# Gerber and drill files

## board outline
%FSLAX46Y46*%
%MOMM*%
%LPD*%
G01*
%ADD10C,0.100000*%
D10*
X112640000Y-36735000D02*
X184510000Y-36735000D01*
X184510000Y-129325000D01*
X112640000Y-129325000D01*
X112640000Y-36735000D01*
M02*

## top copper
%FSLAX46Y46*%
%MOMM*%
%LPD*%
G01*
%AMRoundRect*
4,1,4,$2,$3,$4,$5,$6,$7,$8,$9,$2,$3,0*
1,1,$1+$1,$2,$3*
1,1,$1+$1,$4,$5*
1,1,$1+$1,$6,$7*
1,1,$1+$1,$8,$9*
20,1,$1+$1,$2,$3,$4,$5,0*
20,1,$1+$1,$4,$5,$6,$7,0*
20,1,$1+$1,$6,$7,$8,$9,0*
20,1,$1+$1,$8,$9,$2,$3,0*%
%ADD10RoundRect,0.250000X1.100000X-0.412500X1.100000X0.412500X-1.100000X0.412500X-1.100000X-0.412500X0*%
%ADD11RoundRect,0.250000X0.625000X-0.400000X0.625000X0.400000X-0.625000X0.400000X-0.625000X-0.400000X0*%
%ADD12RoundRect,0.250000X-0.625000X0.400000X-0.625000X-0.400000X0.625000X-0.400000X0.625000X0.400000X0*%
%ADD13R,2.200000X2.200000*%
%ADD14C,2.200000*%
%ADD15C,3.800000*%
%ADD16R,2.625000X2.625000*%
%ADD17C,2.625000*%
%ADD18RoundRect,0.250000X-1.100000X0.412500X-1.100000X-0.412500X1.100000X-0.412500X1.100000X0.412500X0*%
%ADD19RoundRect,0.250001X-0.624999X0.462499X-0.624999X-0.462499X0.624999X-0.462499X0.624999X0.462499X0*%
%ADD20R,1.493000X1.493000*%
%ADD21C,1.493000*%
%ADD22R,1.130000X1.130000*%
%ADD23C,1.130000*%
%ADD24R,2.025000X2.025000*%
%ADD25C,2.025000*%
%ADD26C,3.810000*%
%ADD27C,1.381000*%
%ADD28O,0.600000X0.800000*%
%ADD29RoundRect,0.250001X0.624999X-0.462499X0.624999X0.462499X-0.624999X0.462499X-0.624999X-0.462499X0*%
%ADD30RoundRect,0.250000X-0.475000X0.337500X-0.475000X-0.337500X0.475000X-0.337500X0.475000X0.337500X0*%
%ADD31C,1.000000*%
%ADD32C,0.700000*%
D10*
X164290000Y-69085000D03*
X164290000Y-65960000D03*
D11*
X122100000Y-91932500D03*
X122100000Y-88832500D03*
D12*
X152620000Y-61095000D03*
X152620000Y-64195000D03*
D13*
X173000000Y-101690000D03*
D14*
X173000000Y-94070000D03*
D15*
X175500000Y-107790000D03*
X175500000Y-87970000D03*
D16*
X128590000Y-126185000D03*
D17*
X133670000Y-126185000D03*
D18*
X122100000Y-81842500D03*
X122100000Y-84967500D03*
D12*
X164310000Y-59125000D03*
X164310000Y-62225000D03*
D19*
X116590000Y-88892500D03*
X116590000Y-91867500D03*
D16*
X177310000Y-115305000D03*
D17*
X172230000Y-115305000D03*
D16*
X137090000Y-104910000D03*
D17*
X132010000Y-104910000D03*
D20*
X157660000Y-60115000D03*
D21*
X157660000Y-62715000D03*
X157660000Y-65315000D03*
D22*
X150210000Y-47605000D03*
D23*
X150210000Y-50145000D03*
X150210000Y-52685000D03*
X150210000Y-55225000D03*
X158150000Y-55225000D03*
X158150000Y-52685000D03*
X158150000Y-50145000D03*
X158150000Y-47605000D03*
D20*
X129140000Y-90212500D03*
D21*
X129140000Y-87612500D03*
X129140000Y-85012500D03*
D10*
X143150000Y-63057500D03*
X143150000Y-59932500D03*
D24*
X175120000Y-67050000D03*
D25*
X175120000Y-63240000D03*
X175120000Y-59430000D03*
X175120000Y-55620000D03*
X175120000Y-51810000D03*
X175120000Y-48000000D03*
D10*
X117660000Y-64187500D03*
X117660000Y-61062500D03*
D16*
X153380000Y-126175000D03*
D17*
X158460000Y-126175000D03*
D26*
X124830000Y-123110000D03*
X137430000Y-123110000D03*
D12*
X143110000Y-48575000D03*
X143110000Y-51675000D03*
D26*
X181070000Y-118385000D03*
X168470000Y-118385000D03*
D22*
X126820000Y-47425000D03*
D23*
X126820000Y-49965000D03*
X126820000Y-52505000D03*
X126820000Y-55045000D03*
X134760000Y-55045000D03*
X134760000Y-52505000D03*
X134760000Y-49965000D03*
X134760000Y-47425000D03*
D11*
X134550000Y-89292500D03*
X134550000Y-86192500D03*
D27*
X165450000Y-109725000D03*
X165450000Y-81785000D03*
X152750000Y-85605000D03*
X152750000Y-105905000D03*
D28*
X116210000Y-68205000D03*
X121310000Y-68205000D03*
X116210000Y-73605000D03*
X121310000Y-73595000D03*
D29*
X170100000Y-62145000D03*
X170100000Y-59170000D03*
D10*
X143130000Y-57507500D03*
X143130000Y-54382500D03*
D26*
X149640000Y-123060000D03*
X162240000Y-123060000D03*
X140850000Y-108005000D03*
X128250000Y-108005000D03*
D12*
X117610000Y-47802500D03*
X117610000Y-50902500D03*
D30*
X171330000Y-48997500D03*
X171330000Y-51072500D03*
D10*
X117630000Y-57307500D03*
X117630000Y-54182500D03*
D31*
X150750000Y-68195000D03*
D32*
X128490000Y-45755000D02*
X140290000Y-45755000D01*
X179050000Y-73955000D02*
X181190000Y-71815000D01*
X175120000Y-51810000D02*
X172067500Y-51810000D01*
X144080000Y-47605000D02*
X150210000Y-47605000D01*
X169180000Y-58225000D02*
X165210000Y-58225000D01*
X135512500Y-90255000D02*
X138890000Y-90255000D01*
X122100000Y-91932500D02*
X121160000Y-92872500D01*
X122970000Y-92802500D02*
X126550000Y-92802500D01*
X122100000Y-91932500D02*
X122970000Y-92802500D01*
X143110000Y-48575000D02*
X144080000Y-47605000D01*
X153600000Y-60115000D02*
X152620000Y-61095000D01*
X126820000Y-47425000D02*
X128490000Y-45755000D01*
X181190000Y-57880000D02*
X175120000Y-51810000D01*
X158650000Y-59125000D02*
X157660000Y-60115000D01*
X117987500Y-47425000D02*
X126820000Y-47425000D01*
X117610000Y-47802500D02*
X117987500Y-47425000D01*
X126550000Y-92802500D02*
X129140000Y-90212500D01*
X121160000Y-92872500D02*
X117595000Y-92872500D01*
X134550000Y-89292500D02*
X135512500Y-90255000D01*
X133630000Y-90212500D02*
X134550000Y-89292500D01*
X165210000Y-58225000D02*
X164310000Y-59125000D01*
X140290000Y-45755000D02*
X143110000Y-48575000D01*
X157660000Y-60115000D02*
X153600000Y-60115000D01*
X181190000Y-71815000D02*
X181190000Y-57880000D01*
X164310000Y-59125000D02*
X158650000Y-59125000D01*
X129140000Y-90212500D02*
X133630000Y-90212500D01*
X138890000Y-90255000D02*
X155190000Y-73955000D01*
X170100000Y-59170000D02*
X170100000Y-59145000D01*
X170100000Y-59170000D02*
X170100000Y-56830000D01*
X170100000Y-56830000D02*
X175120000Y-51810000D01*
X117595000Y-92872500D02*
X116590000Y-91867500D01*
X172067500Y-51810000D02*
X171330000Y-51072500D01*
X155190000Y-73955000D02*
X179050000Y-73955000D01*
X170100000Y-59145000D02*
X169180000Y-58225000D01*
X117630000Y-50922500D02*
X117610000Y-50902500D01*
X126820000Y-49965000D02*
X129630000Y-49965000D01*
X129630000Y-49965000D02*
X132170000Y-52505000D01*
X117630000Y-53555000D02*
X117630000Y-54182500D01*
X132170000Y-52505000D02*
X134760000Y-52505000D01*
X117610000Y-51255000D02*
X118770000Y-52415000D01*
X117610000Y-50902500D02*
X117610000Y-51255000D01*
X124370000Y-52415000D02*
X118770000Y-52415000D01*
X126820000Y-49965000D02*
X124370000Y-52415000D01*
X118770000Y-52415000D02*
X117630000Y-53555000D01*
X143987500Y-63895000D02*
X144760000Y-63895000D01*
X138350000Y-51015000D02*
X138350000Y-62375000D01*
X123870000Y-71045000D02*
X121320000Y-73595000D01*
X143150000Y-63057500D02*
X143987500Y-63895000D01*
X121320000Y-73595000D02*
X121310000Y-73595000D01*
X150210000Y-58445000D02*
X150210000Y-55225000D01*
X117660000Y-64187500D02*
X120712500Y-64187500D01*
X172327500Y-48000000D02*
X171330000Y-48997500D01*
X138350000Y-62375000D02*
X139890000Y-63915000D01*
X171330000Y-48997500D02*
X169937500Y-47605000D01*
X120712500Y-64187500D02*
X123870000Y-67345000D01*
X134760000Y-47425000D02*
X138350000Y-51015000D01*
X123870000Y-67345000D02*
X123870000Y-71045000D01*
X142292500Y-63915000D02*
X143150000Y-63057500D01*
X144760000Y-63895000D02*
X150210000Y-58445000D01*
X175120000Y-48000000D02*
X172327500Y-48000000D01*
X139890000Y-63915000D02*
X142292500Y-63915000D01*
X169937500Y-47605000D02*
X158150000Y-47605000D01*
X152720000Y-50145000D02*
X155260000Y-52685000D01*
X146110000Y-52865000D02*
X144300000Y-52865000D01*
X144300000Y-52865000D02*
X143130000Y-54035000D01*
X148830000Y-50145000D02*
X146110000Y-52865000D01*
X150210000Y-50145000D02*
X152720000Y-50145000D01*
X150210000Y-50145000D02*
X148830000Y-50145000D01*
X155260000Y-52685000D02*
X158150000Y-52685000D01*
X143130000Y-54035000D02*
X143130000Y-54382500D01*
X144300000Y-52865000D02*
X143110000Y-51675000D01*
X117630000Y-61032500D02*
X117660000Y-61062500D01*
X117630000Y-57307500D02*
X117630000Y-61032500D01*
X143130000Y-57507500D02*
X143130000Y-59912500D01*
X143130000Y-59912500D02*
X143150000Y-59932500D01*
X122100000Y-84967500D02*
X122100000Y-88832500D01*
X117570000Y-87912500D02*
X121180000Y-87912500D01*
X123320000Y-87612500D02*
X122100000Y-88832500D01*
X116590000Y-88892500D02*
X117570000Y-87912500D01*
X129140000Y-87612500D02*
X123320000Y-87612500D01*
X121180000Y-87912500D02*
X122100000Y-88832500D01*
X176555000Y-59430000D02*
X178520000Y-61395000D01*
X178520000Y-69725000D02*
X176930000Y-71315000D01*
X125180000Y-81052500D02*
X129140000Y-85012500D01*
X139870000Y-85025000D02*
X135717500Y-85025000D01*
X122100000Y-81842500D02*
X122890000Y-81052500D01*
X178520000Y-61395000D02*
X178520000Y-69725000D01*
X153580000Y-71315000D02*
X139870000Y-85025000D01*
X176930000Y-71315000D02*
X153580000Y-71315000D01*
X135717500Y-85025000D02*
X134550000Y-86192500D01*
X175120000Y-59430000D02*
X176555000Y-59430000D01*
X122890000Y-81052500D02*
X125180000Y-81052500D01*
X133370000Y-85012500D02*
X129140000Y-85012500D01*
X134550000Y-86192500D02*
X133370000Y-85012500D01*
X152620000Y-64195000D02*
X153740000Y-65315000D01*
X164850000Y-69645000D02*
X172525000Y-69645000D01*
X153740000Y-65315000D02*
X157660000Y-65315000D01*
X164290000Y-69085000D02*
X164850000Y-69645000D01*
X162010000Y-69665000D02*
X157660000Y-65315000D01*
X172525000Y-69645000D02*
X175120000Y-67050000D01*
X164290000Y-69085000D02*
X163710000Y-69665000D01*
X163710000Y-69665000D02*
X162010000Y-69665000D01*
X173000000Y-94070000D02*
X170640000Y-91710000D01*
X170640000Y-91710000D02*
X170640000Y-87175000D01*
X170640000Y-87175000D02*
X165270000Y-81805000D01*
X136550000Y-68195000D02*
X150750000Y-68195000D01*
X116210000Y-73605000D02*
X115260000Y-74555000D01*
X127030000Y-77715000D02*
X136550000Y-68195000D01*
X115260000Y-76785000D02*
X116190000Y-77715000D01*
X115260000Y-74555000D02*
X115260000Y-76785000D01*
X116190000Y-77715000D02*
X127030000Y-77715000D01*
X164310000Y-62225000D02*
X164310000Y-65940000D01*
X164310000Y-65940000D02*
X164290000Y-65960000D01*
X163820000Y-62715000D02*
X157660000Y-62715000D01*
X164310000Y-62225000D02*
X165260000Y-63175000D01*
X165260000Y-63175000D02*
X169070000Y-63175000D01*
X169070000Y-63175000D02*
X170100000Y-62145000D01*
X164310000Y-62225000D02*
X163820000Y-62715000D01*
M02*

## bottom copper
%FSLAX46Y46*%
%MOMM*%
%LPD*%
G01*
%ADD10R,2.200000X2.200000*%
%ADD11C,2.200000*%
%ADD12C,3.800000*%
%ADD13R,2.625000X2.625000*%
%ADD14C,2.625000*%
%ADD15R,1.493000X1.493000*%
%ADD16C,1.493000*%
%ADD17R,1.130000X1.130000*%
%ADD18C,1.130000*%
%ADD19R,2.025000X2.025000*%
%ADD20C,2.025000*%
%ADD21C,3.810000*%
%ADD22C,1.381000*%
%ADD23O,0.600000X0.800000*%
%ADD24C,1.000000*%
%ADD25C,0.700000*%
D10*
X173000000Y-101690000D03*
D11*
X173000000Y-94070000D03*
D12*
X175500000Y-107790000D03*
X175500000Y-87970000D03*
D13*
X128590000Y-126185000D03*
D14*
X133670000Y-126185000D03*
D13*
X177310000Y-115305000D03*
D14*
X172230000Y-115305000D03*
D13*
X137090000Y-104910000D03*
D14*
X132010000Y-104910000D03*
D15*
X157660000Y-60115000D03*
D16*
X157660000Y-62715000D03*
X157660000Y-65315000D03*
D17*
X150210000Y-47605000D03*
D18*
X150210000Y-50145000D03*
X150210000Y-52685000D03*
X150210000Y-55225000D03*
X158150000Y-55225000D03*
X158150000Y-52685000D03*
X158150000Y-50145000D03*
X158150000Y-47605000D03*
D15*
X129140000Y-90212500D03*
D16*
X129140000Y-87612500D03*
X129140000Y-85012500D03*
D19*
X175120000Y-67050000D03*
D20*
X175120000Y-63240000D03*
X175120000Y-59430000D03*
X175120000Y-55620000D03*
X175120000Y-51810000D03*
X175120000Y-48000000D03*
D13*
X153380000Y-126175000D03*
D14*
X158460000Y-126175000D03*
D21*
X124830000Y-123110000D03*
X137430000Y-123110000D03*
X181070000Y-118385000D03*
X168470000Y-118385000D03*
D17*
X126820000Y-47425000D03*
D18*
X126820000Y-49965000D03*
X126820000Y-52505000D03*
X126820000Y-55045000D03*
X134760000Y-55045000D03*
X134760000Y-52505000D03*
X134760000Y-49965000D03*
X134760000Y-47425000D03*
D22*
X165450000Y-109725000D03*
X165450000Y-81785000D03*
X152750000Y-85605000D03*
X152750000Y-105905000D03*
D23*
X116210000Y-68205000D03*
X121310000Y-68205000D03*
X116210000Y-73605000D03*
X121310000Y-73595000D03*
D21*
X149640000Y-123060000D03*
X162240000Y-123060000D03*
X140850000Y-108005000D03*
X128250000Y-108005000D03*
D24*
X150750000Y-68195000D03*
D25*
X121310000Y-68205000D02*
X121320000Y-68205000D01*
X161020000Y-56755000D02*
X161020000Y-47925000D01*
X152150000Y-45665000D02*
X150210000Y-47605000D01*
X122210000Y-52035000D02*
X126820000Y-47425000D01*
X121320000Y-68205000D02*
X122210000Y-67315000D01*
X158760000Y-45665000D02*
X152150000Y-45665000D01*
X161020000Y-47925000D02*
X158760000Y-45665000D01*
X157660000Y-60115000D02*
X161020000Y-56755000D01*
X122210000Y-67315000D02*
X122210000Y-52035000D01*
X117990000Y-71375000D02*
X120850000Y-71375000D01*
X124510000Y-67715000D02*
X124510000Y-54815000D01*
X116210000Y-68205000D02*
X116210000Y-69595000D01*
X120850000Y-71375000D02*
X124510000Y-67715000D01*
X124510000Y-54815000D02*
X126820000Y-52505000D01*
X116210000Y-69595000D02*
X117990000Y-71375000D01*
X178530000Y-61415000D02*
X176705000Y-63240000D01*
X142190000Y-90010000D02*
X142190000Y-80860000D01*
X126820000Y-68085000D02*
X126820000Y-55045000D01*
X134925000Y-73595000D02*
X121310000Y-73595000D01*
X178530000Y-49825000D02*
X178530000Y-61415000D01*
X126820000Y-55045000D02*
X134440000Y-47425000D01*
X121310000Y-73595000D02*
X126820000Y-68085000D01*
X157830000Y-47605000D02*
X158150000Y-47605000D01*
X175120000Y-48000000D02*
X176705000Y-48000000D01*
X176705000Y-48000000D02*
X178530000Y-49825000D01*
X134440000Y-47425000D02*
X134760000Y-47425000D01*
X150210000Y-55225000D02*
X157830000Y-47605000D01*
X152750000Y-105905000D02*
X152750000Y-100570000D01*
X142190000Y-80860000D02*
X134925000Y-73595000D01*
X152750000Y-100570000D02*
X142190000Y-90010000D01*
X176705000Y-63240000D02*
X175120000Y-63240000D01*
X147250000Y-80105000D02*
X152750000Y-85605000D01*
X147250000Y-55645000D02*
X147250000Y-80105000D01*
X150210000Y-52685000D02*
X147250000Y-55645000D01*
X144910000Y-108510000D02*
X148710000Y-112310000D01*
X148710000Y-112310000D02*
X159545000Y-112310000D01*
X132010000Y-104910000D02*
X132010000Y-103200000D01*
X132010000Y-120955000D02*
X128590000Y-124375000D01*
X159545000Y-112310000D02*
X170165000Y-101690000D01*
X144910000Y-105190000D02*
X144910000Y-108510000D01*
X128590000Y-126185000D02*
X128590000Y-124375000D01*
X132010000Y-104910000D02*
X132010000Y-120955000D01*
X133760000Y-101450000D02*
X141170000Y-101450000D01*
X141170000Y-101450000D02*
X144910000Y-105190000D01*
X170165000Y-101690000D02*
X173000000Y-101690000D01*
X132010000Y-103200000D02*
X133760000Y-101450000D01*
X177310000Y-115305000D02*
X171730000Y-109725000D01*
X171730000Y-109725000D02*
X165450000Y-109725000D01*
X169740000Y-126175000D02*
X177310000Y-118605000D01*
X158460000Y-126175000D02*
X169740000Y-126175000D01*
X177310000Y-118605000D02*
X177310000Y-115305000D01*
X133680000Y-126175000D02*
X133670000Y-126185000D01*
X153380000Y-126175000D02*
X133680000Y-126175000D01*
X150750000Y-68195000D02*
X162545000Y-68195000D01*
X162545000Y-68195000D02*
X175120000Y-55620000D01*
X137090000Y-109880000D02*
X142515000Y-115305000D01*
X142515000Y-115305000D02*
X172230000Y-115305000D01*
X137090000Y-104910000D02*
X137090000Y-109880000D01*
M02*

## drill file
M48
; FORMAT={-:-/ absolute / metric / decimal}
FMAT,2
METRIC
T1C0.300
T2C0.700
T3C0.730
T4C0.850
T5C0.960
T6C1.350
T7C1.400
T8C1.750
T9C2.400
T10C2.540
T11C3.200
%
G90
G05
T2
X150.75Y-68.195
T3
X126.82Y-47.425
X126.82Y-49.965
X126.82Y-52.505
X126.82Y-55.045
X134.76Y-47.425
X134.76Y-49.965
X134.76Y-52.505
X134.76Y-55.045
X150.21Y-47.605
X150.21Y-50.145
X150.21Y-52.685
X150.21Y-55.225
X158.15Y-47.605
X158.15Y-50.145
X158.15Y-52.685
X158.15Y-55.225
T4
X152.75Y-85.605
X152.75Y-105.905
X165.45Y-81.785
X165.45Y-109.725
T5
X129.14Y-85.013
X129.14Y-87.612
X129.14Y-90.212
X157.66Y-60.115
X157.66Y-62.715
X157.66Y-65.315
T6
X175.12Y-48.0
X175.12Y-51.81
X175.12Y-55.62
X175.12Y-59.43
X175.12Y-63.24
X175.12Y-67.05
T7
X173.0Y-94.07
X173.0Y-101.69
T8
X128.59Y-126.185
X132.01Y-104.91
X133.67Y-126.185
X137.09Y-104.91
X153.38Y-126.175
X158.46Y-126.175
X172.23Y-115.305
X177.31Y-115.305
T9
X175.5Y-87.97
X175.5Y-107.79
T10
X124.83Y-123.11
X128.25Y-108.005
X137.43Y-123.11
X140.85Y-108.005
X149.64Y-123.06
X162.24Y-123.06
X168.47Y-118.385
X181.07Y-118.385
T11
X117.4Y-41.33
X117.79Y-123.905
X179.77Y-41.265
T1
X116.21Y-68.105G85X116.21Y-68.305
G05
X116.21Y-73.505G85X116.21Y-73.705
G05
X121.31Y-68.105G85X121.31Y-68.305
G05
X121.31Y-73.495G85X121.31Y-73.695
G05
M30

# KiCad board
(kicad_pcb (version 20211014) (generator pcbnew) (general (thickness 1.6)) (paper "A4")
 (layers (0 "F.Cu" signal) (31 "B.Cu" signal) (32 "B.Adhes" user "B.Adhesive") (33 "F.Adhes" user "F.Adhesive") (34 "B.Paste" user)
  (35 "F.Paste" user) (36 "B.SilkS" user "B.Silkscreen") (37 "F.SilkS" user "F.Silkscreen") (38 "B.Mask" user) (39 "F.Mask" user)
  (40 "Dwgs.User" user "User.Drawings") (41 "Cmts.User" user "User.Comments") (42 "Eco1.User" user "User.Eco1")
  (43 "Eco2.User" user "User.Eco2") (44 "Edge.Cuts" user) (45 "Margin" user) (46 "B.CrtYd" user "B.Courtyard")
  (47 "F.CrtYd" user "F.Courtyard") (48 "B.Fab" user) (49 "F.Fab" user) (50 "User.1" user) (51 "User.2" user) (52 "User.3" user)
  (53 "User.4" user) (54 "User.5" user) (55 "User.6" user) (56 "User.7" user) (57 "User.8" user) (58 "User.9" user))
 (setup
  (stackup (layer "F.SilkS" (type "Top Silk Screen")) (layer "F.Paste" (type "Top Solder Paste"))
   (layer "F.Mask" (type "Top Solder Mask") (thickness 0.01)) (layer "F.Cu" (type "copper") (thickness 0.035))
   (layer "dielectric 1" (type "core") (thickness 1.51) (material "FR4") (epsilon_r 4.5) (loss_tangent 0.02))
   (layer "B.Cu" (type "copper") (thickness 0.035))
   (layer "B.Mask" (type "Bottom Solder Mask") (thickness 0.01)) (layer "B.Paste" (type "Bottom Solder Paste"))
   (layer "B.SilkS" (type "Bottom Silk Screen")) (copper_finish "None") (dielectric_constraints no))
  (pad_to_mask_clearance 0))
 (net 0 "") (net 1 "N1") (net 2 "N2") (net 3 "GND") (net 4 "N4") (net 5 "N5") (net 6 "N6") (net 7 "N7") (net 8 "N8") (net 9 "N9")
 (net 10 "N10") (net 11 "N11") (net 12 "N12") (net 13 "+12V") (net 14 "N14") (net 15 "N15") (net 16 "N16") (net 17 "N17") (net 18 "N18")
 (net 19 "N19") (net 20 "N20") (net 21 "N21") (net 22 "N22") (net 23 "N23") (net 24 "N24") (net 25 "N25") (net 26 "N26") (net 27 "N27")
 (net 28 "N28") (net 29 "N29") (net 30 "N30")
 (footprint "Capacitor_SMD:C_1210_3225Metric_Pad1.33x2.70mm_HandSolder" (layer "F.Cu") (at 164.29 67.5225 90)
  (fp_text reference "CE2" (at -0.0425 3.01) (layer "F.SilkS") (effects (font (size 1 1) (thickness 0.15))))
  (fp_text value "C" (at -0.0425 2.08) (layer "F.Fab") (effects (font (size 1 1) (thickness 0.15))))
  (pad "1" smd roundrect (at -1.5625 0 90) (size 1.325 2.7) (layers "F.Cu" "F.Paste" "F.Mask") (roundrect_rratio 0.1886792453) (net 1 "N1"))
  (pad "2" smd roundrect (at 1.5625 0 90) (size 1.325 2.7) (layers "F.Cu" "F.Paste" "F.Mask") (roundrect_rratio 0.1886792453) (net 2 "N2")))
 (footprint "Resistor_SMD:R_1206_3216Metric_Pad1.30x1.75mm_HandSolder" (layer "F.Cu") (at 122.1 90.3825 90)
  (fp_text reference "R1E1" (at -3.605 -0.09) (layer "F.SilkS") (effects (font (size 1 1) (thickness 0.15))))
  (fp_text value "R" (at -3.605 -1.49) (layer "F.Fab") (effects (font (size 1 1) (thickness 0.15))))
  (pad "1" smd roundrect (at -1.55 0 90) (size 1.3 1.75) (layers "F.Cu" "F.Paste" "F.Mask") (roundrect_rratio 0.1923076923) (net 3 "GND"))
  (pad "2" smd roundrect (at 1.55 0 90) (size 1.3 1.75) (layers "F.Cu" "F.Paste" "F.Mask") (roundrect_rratio 0.1923076923) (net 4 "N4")))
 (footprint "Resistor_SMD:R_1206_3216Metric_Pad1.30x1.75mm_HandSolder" (layer "F.Cu") (at 152.62 62.645 -90)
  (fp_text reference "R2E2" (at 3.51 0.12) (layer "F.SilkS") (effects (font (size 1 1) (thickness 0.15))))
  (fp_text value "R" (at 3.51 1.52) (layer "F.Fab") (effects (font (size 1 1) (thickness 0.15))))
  (pad "1" smd roundrect (at -1.55 0 270) (size 1.3 1.75) (layers "F.Cu" "F.Paste" "F.Mask") (roundrect_rratio 0.1923076923) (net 3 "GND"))
  (pad "2" smd roundrect (at 1.55 0 270) (size 1.3 1.75) (layers "F.Cu" "F.Paste" "F.Mask") (roundrect_rratio 0.1923076923) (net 1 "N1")))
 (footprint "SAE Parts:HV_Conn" (layer "F.Cu") (at 173 101.69 90)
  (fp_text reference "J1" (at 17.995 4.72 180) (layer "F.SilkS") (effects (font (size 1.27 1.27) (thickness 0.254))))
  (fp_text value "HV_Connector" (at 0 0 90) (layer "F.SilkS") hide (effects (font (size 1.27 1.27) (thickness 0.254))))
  (pad "1" thru_hole rect (at 0 0 90) (size 2.2 2.2) (drill 1.4) (layers *.Cu *.Mask) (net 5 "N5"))
  (pad "2" thru_hole circle (at 7.62 0 90) (size 2.2 2.2) (drill 1.4) (layers *.Cu *.Mask) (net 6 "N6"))
  (pad "3" thru_hole circle (at -6.1 2.5 90) (size 3.8 3.8) (drill 2.4) (layers *.Cu *.Mask))
  (pad "4" thru_hole circle (at 13.72 2.5 90) (size 3.8 3.8) (drill 2.4) (layers *.Cu *.Mask)))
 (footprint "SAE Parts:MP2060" (layer "F.Cu") (at 128.59 126.185)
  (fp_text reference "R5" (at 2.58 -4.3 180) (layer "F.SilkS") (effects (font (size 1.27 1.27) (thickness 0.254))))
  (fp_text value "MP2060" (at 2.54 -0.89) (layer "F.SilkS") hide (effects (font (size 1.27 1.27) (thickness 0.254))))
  (pad "1" thru_hole rect (at 0 0) (size 2.625 2.625) (drill 1.75) (layers *.Cu *.Mask) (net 5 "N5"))
  (pad "2" thru_hole circle (at 5.08 0) (size 2.625 2.625) (drill 1.75) (layers *.Cu *.Mask) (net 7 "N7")))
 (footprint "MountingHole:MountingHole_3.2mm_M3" (layer "F.Cu") (at 117.4 41.33)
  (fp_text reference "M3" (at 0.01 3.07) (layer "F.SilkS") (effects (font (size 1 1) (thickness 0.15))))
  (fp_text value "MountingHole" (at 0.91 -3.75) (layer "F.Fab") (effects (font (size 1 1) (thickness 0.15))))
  (pad "" np_thru_hole circle (at 0 0) (size 3.2 3.2) (drill 3.2) (layers *.Cu *.Mask)))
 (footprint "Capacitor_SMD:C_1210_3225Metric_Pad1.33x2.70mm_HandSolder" (layer "F.Cu") (at 122.1 83.405 -90)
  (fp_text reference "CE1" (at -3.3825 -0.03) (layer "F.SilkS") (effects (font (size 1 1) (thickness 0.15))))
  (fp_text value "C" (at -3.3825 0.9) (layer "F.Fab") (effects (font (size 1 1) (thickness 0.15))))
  (pad "1" smd roundrect (at -1.5625 0 270) (size 1.325 2.7) (layers "F.Cu" "F.Paste" "F.Mask") (roundrect_rratio 0.1886792453) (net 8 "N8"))
  (pad "2" smd roundrect (at 1.5625 0 270) (size 1.325 2.7) (layers "F.Cu" "F.Paste" "F.Mask") (roundrect_rratio 0.1886792453) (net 4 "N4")))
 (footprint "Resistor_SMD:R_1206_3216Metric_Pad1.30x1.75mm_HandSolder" (layer "F.Cu") (at 164.31 60.675 -90)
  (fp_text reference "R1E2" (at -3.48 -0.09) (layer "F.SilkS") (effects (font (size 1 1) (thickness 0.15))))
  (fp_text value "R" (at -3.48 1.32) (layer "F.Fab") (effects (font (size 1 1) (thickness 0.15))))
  (pad "1" smd roundrect (at -1.55 0 270) (size 1.3 1.75) (layers "F.Cu" "F.Paste" "F.Mask") (roundrect_rratio 0.1923076923) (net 3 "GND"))
  (pad "2" smd roundrect (at 1.55 0 270) (size 1.3 1.75) (layers "F.Cu" "F.Paste" "F.Mask") (roundrect_rratio 0.1923076923) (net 2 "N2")))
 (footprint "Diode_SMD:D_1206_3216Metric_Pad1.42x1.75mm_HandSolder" (layer "F.Cu") (at 116.59 90.38 -90)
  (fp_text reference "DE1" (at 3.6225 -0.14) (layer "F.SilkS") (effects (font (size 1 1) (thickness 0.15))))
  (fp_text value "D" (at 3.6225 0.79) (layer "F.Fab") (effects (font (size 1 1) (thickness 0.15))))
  (pad "1" smd roundrect (at -1.4875 0 270) (size 1.425 1.75) (layers "F.Cu" "F.Paste" "F.Mask") (roundrect_rratio 0.1754392982)
   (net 4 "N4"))
  (pad "2" smd roundrect (at 1.4875 0 270) (size 1.425 1.75) (layers "F.Cu" "F.Paste" "F.Mask") (roundrect_rratio 0.1754392982)
   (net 3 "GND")))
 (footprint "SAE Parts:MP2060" (layer "F.Cu") (at 177.31 115.305 180)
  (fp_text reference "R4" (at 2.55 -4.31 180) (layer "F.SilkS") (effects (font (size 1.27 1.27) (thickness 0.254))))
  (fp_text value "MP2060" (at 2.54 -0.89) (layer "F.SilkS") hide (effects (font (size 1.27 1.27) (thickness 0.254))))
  (pad "1" thru_hole rect (at 0 0 180) (size 2.625 2.625) (drill 1.75) (layers *.Cu *.Mask) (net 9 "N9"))
  (pad "2" thru_hole circle (at 5.08 0 180) (size 2.625 2.625) (drill 1.75) (layers *.Cu *.Mask) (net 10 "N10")))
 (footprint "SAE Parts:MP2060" (layer "F.Cu") (at 137.09 104.91 180)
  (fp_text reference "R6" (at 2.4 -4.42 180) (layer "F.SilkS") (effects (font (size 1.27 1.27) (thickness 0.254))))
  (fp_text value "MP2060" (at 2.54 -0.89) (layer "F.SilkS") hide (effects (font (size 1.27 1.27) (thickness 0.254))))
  (pad "1" thru_hole rect (at 0 0 180) (size 2.625 2.625) (drill 1.75) (layers *.Cu *.Mask) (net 10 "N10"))
  (pad "2" thru_hole circle (at 5.08 0 180) (size 2.625 2.625) (drill 1.75) (layers *.Cu *.Mask) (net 5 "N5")))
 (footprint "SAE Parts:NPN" (layer "F.Cu") (at 157.66 60.115 -90)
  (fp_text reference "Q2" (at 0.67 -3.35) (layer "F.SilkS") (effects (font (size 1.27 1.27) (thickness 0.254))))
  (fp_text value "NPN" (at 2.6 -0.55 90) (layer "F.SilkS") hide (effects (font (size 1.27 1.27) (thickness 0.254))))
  (pad "1" thru_hole rect (at 0 0 270) (size 1.493 1.493) (drill 0.96) (layers *.Cu *.Mask) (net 3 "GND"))
  (pad "2" thru_hole circle (at 2.6 0 270) (size 1.493 1.493) (drill 0.96) (layers *.Cu *.Mask) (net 2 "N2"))
  (pad "3" thru_hole circle (at 5.2 0 270) (size 1.493 1.493) (drill 0.96) (layers *.Cu *.Mask) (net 1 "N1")))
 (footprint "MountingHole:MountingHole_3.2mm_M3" (layer "F.Cu") (at 117.79 123.905)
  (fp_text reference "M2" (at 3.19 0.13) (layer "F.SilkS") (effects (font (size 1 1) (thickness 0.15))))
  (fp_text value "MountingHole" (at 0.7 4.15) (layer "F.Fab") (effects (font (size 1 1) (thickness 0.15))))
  (pad "" np_thru_hole circle (at 0 0) (size 3.2 3.2) (drill 3.2) (layers *.Cu *.Mask)))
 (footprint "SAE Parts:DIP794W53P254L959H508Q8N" (layer "F.Cu") (at 154.18 51.415)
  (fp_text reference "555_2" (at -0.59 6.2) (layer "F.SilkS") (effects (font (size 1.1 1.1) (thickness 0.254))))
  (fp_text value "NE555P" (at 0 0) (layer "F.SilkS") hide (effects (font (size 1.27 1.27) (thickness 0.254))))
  (pad "1" thru_hole rect (at -3.97 -3.81) (size 1.13 1.13) (drill 0.73) (layers *.Cu *.Mask) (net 3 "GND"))
  (pad "2" thru_hole circle (at -3.97 -1.27) (size 1.13 1.13) (drill 0.73) (layers *.Cu *.Mask) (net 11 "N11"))
  (pad "3" thru_hole circle (at -3.97 1.27) (size 1.13 1.13) (drill 0.73) (layers *.Cu *.Mask) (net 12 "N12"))
  (pad "4" thru_hole circle (at -3.97 3.81) (size 1.13 1.13) (drill 0.73) (layers *.Cu *.Mask) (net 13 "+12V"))
  (pad "5" thru_hole circle (at 3.97 3.81) (size 1.13 1.13) (drill 0.73) (layers *.Cu *.Mask) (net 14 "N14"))
  (pad "6" thru_hole circle (at 3.97 1.27) (size 1.13 1.13) (drill 0.73) (layers *.Cu *.Mask) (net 11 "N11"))
  (pad "7" thru_hole circle (at 3.97 -1.27) (size 1.13 1.13) (drill 0.73) (layers *.Cu *.Mask) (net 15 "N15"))
  (pad "8" thru_hole circle (at 3.97 -3.81) (size 1.13 1.13) (drill 0.73) (layers *.Cu *.Mask) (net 13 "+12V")))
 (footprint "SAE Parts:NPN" (layer "F.Cu") (at 129.14 90.2125 90)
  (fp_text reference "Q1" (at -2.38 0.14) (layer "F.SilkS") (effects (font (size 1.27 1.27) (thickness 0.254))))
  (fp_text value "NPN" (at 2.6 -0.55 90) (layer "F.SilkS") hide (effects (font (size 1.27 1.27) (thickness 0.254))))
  (pad "1" thru_hole rect (at 0 0 90) (size 1.493 1.493) (drill 0.96) (layers *.Cu *.Mask) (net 3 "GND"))
  (pad "2" thru_hole circle (at 2.6 0 90) (size 1.493 1.493) (drill 0.96) (layers *.Cu *.Mask) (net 4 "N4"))
  (pad "3" thru_hole circle (at 5.2 0 90) (size 1.493 1.493) (drill 0.96) (layers *.Cu *.Mask) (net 8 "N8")))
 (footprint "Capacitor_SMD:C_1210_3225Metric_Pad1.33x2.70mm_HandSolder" (layer "F.Cu") (at 143.15 61.495 90)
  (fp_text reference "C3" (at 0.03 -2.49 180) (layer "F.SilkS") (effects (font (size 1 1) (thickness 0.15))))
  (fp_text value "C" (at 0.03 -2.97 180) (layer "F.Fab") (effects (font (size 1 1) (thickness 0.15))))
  (pad "1" smd roundrect (at -1.5625 0 90) (size 1.325 2.7) (layers "F.Cu" "F.Paste" "F.Mask") (roundrect_rratio 0.1886792453)
   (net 13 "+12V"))
  (pad "2" smd roundrect (at 1.5625 0 90) (size 1.325 2.7) (layers "F.Cu" "F.Paste" "F.Mask") (roundrect_rratio 0.1886792453) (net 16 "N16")))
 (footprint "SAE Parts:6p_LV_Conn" (layer "F.Cu") (at 175.12 67.05 -90)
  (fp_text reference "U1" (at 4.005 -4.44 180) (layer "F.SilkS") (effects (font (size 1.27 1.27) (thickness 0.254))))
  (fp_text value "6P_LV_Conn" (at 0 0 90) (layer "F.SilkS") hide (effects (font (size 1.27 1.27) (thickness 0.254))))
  (pad "1" thru_hole rect (at 0 0 270) (size 2.025 2.025) (drill 1.35) (layers *.Cu *.Mask) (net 1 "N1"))
  (pad "2" thru_hole circle (at -3.81 0 270) (size 2.025 2.025) (drill 1.35) (layers *.Cu *.Mask) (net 13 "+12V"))
  (pad "3" thru_hole circle (at -7.62 0 270) (size 2.025 2.025) (drill 1.35) (layers *.Cu *.Mask) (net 8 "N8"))
  (pad "4" thru_hole circle (at -11.43 0 270) (size 2.025 2.025) (drill 1.35) (layers *.Cu *.Mask) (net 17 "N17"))
  (pad "5" thru_hole circle (at -15.24 0 270) (size 2.025 2.025) (drill 1.35) (layers *.Cu *.Mask) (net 3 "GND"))
  (pad "6" thru_hole circle (at -19.05 0 270) (size 2.025 2.025) (drill 1.35) (layers *.Cu *.Mask) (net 13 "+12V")))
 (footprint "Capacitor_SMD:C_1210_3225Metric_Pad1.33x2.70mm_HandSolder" (layer "F.Cu") (at 117.66 62.625 90)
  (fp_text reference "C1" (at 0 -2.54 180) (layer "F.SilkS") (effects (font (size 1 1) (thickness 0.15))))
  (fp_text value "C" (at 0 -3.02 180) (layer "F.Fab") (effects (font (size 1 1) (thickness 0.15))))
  (pad "1" smd roundrect (at -1.5625 0 90) (size 1.325 2.7) (layers "F.Cu" "F.Paste" "F.Mask") (roundrect_rratio 0.1886792453)
   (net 13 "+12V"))
  (pad "2" smd roundrect (at 1.5625 0 90) (size 1.325 2.7) (layers "F.Cu" "F.Paste" "F.Mask") (roundrect_rratio 0.1886792453) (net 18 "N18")))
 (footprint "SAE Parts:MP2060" (layer "F.Cu") (at 153.38 126.175)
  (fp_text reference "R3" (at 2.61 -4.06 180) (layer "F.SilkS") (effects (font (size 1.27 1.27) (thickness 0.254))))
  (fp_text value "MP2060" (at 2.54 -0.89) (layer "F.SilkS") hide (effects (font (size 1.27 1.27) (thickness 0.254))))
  (pad "1" thru_hole rect (at 0 0) (size 2.625 2.625) (drill 1.75) (layers *.Cu *.Mask) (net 7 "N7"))
  (pad "2" thru_hole circle (at 5.08 0) (size 2.625 2.625) (drill 1.75) (layers *.Cu *.Mask) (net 9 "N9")))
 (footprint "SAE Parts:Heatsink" (layer "F.Cu") (at 124.83 123.11)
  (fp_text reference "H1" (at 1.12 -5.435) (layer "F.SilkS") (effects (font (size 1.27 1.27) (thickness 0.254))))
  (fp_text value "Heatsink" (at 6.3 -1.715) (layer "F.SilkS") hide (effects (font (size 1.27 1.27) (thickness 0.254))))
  (pad "1" thru_hole circle (at 0 0) (size 3.81 3.81) (drill 2.54) (layers *.Cu *.Mask) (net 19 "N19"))
  (pad "2" thru_hole circle (at 12.6 0) (size 3.81 3.81) (drill 2.54) (layers *.Cu *.Mask) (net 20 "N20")))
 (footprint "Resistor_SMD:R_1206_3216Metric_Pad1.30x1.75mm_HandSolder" (layer "F.Cu") (at 143.11 50.125 -90)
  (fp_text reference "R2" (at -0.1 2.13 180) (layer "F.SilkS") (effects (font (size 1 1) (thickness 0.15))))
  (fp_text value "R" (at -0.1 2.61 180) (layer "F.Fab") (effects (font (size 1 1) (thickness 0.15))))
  (pad "1" smd roundrect (at -1.55 0 270) (size 1.3 1.75) (layers "F.Cu" "F.Paste" "F.Mask") (roundrect_rratio 0.1923076923) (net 3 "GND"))
  (pad "2" smd roundrect (at 1.55 0 270) (size 1.3 1.75) (layers "F.Cu" "F.Paste" "F.Mask") (roundrect_rratio 0.1923076923) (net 11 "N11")))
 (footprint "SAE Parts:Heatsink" (layer "F.Cu") (at 181.07 118.385 180)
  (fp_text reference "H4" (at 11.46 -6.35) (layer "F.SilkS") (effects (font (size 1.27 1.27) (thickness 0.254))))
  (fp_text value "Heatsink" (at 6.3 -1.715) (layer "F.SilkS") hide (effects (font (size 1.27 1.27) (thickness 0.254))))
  (pad "1" thru_hole circle (at 0 0 180) (size 3.81 3.81) (drill 2.54) (layers *.Cu *.Mask) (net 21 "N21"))
  (pad "2" thru_hole circle (at 12.6 0 180) (size 3.81 3.81) (drill 2.54) (layers *.Cu *.Mask) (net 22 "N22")))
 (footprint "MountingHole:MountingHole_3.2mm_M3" (layer "F.Cu") (at 179.77 41.265)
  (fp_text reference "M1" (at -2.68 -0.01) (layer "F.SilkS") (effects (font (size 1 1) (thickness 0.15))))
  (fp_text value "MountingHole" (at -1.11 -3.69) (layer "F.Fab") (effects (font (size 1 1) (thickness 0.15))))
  (pad "" np_thru_hole circle (at 0 0) (size 3.2 3.2) (drill 3.2) (layers *.Cu *.Mask)))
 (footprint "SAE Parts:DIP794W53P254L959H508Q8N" (layer "F.Cu") (at 130.79 51.235)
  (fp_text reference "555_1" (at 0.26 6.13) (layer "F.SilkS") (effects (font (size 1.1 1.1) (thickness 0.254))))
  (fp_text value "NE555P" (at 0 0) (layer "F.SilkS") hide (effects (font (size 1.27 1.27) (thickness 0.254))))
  (pad "1" thru_hole rect (at -3.97 -3.81) (size 1.13 1.13) (drill 0.73) (layers *.Cu *.Mask) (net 3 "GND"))
  (pad "2" thru_hole circle (at -3.97 -1.27) (size 1.13 1.13) (drill 0.73) (layers *.Cu *.Mask) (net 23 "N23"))
  (pad "3" thru_hole circle (at -3.97 1.27) (size 1.13 1.13) (drill 0.73) (layers *.Cu *.Mask) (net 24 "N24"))
  (pad "4" thru_hole circle (at -3.97 3.81) (size 1.13 1.13) (drill 0.73) (layers *.Cu *.Mask) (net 13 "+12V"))
  (pad "5" thru_hole circle (at 3.97 3.81) (size 1.13 1.13) (drill 0.73) (layers *.Cu *.Mask) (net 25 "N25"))
  (pad "6" thru_hole circle (at 3.97 1.27) (size 1.13 1.13) (drill 0.73) (layers *.Cu *.Mask) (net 23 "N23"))
  (pad "7" thru_hole circle (at 3.97 -1.27) (size 1.13 1.13) (drill 0.73) (layers *.Cu *.Mask) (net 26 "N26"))
  (pad "8" thru_hole circle (at 3.97 -3.81) (size 1.13 1.13) (drill 0.73) (layers *.Cu *.Mask) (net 13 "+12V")))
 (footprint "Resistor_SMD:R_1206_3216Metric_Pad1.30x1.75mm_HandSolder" (layer "F.Cu") (at 134.55 87.7425 90)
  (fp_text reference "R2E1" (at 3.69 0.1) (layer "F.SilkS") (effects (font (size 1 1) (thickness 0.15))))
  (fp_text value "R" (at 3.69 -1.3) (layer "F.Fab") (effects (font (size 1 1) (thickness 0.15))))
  (pad "1" smd roundrect (at -1.55 0 90) (size 1.3 1.75) (layers "F.Cu" "F.Paste" "F.Mask") (roundrect_rratio 0.1923076923) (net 3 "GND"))
  (pad "2" smd roundrect (at 1.55 0 90) (size 1.3 1.75) (layers "F.Cu" "F.Paste" "F.Mask") (roundrect_rratio 0.1923076923) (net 8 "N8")))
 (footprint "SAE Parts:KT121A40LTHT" (layer "F.Cu") (at 165.45 109.725 90)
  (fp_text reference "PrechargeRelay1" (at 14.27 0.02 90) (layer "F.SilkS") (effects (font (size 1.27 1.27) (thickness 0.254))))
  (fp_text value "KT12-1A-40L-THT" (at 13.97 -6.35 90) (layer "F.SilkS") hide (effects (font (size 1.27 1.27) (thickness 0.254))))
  (pad "1" thru_hole circle (at 0 0 90) (size 1.381 1.381) (drill 0.85) (layers *.Cu *.Mask) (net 9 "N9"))
  (pad "2" thru_hole circle (at 27.94 0 90) (size 1.381 1.381) (drill 0.85) (layers *.Cu *.Mask) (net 6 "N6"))
  (pad "3" thru_hole circle (at 24.12 -12.7 90) (size 1.381 1.381) (drill 0.85) (layers *.Cu *.Mask) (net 12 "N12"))
  (pad "4" thru_hole circle (at 3.82 -12.7 90) (size 1.381 1.381) (drill 0.85) (layers *.Cu *.Mask) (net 13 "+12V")))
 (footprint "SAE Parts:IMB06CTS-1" (layer "F.Cu") (at 118.91 72.105)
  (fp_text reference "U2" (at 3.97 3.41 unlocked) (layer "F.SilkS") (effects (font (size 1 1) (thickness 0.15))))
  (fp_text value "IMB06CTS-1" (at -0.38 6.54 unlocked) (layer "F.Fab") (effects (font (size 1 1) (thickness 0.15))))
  (pad "1" thru_hole oval (at -2.7 -3.9) (size 0.6 0.8) (drill oval 0.3 0.5) (layers *.Cu *.Mask) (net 24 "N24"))
  (pad "2" thru_hole oval (at 2.4 -3.9) (size 0.6 0.8) (drill oval 0.3 0.5) (layers *.Cu *.Mask) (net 3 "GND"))
  (pad "3" thru_hole oval (at -2.7 1.5) (size 0.6 0.8) (drill oval 0.3 0.5) (layers *.Cu *.Mask) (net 17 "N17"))
  (pad "4" thru_hole oval (at 2.4 1.49) (size 0.6 0.8) (drill oval 0.3 0.5) (layers *.Cu *.Mask) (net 13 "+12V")))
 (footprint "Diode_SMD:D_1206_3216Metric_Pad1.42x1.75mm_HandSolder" (layer "F.Cu") (at 170.1 60.6575 90)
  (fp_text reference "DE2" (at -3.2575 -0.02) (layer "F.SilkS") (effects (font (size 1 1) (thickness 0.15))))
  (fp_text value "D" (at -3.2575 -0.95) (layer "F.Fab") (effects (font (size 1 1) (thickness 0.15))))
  (pad "1" smd roundrect (at -1.4875 0 90) (size 1.425 1.75) (layers "F.Cu" "F.Paste" "F.Mask") (roundrect_rratio 0.1754392982) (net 2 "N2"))
  (pad "2" smd roundrect (at 1.4875 0 90) (size 1.425 1.75) (layers "F.Cu" "F.Paste" "F.Mask") (roundrect_rratio 0.1754392982) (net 3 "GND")))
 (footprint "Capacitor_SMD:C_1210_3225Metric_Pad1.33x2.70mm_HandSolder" (layer "F.Cu") (at 143.13 55.945 90)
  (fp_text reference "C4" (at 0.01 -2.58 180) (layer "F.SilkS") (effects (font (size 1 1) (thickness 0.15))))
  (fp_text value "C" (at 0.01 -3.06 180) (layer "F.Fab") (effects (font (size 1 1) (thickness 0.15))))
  (pad "1" smd roundrect (at -1.5625 0 90) (size 1.325 2.7) (layers "F.Cu" "F.Paste" "F.Mask") (roundrect_rratio 0.1886792453)
   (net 16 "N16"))
  (pad "2" smd roundrect (at 1.5625 0 90) (size 1.325 2.7) (layers "F.Cu" "F.Paste" "F.Mask") (roundrect_rratio 0.1886792453) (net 11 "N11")))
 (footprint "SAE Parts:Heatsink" (layer "F.Cu") (at 149.64 123.06)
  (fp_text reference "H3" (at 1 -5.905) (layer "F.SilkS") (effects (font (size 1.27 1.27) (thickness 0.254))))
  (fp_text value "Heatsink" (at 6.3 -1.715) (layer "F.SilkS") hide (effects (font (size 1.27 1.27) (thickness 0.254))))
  (pad "1" thru_hole circle (at 0 0) (size 3.81 3.81) (drill 2.54) (layers *.Cu *.Mask) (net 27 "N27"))
  (pad "2" thru_hole circle (at 12.6 0) (size 3.81 3.81) (drill 2.54) (layers *.Cu *.Mask) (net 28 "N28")))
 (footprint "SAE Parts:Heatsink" (layer "F.Cu") (at 140.85 108.005 180)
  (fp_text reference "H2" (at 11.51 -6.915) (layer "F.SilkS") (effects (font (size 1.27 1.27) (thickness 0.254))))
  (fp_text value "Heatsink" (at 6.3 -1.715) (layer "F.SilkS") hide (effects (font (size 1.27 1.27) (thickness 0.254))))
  (pad "1" thru_hole circle (at 0 0 180) (size 3.81 3.81) (drill 2.54) (layers *.Cu *.Mask) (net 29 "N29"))
  (pad "2" thru_hole circle (at 12.6 0 180) (size 3.81 3.81) (drill 2.54) (layers *.Cu *.Mask) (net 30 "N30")))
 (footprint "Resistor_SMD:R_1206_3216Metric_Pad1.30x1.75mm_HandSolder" (layer "F.Cu") (at 117.61 49.3525 -90)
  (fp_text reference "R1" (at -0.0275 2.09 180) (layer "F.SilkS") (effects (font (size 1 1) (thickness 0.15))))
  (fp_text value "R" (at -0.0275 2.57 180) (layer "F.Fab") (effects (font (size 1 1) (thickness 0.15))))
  (pad "1" smd roundrect (at -1.55 0 270) (size 1.3 1.75) (layers "F.Cu" "F.Paste" "F.Mask") (roundrect_rratio 0.1923076923) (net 3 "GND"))
  (pad "2" smd roundrect (at 1.55 0 270) (size 1.3 1.75) (layers "F.Cu" "F.Paste" "F.Mask") (roundrect_rratio 0.1923076923) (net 23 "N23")))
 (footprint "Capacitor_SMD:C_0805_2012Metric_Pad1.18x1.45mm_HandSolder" (layer "F.Cu") (at 171.33 50.035 -90)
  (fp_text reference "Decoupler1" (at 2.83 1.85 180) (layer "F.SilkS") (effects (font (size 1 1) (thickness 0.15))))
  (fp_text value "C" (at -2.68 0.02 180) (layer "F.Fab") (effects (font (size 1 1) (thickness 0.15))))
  (pad "1" smd roundrect (at -1.0375 0 270) (size 1.175 1.45) (layers "F.Cu" "F.Paste" "F.Mask") (roundrect_rratio 0.2127659574)
   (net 13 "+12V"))
  (pad "2" smd roundrect (at 1.0375 0 270) (size 1.175 1.45) (layers "F.Cu" "F.Paste" "F.Mask") (roundrect_rratio 0.2127659574)
   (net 3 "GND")))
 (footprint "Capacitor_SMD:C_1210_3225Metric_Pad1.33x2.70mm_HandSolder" (layer "F.Cu") (at 117.63 55.745 90)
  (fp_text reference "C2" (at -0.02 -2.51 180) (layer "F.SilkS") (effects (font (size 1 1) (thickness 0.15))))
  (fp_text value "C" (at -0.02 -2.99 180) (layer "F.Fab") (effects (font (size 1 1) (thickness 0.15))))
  (pad "1" smd roundrect (at -1.5625 0 90) (size 1.325 2.7) (layers "F.Cu" "F.Paste" "F.Mask") (roundrect_rratio 0.1886792453)
   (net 18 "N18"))
  (pad "2" smd roundrect (at 1.5625 0 90) (size 1.325 2.7) (layers "F.Cu" "F.Paste" "F.Mask") (roundrect_rratio 0.1886792453) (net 23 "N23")))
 (gr_rect (start 184.51 129.325) (end 112.64 36.735) (layer "Edge.Cuts") (width 0.1) (fill none))
 (segment (start 128.49 45.755) (end 140.29 45.755) (width 0.7) (layer "F.Cu") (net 3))
 (segment (start 179.05 73.955) (end 181.19 71.815) (width 0.7) (layer "F.Cu") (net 3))
 (segment (start 175.12 51.81) (end 172.0675 51.81) (width 0.7) (layer "F.Cu") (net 3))
 (segment (start 144.08 47.605) (end 150.21 47.605) (width 0.7) (layer "F.Cu") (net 3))
 (segment (start 169.18 58.225) (end 165.21 58.225) (width 0.7) (layer "F.Cu") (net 3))
 (segment (start 135.5125 90.255) (end 138.89 90.255) (width 0.7) (layer "F.Cu") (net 3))
 (segment (start 122.1 91.9325) (end 121.16 92.8725) (width 0.7) (layer "F.Cu") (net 3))
 (segment (start 122.97 92.8025) (end 126.55 92.8025) (width 0.7) (layer "F.Cu") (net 3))
 (segment (start 122.1 91.9325) (end 122.97 92.8025) (width 0.7) (layer "F.Cu") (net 3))
 (segment (start 143.11 48.575) (end 144.08 47.605) (width 0.7) (layer "F.Cu") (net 3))
 (segment (start 153.6 60.115) (end 152.62 61.095) (width 0.7) (layer "F.Cu") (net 3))
 (segment (start 126.82 47.425) (end 128.49 45.755) (width 0.7) (layer "F.Cu") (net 3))
 (segment (start 181.19 57.88) (end 175.12 51.81) (width 0.7) (layer "F.Cu") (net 3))
 (segment (start 158.65 59.125) (end 157.66 60.115) (width 0.7) (layer "F.Cu") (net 3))
 (segment (start 117.9875 47.425) (end 126.82 47.425) (width 0.7) (layer "F.Cu") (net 3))
 (segment (start 117.61 47.8025) (end 117.9875 47.425) (width 0.7) (layer "F.Cu") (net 3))
 (segment (start 126.55 92.8025) (end 129.14 90.2125) (width 0.7) (layer "F.Cu") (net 3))
 (segment (start 121.16 92.8725) (end 117.595 92.8725) (width 0.7) (layer "F.Cu") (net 3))
 (segment (start 134.55 89.2925) (end 135.5125 90.255) (width 0.7) (layer "F.Cu") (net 3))
 (segment (start 133.63 90.2125) (end 134.55 89.2925) (width 0.7) (layer "F.Cu") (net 3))
 (segment (start 165.21 58.225) (end 164.31 59.125) (width 0.7) (layer "F.Cu") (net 3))
 (segment (start 140.29 45.755) (end 143.11 48.575) (width 0.7) (layer "F.Cu") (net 3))
 (segment (start 157.66 60.115) (end 153.6 60.115) (width 0.7) (layer "F.Cu") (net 3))
 (segment (start 181.19 71.815) (end 181.19 57.88) (width 0.7) (layer "F.Cu") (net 3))
 (segment (start 164.31 59.125) (end 158.65 59.125) (width 0.7) (layer "F.Cu") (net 3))
 (segment (start 129.14 90.2125) (end 133.63 90.2125) (width 0.7) (layer "F.Cu") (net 3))
 (segment (start 138.89 90.255) (end 155.19 73.955) (width 0.7) (layer "F.Cu") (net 3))
 (segment (start 170.1 59.17) (end 170.1 59.145) (width 0.7) (layer "F.Cu") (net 3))
 (segment (start 170.1 59.17) (end 170.1 56.83) (width 0.7) (layer "F.Cu") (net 3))
 (segment (start 170.1 56.83) (end 175.12 51.81) (width 0.7) (layer "F.Cu") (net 3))
 (segment (start 117.595 92.8725) (end 116.59 91.8675) (width 0.7) (layer "F.Cu") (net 3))
 (segment (start 172.0675 51.81) (end 171.33 51.0725) (width 0.7) (layer "F.Cu") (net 3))
 (segment (start 155.19 73.955) (end 179.05 73.955) (width 0.7) (layer "F.Cu") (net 3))
 (segment (start 170.1 59.145) (end 169.18 58.225) (width 0.7) (layer "F.Cu") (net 3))
 (segment (start 121.31 68.205) (end 121.32 68.205) (width 0.7) (layer "B.Cu") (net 3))
 (segment (start 161.02 56.755) (end 161.02 47.925) (width 0.7) (layer "B.Cu") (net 3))
 (segment (start 152.15 45.665) (end 150.21 47.605) (width 0.7) (layer "B.Cu") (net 3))
 (segment (start 122.21 52.035) (end 126.82 47.425) (width 0.7) (layer "B.Cu") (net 3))
 (segment (start 121.32 68.205) (end 122.21 67.315) (width 0.7) (layer "B.Cu") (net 3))
 (segment (start 158.76 45.665) (end 152.15 45.665) (width 0.7) (layer "B.Cu") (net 3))
 (segment (start 161.02 47.925) (end 158.76 45.665) (width 0.7) (layer "B.Cu") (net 3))
 (segment (start 157.66 60.115) (end 161.02 56.755) (width 0.7) (layer "B.Cu") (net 3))
 (segment (start 122.21 67.315) (end 122.21 52.035) (width 0.7) (layer "B.Cu") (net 3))
 (segment (start 117.63 50.9225) (end 117.61 50.9025) (width 0.7) (layer "F.Cu") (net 23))
 (segment (start 126.82 49.965) (end 129.63 49.965) (width 0.7) (layer "F.Cu") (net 23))
 (segment (start 129.63 49.965) (end 132.17 52.505) (width 0.7) (layer "F.Cu") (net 23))
 (segment (start 117.63 53.555) (end 117.63 54.1825) (width 0.7) (layer "F.Cu") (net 23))
 (segment (start 132.17 52.505) (end 134.76 52.505) (width 0.7) (layer "F.Cu") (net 23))
 (segment (start 117.61 51.255) (end 118.77 52.415) (width 0.7) (layer "F.Cu") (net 23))
 (segment (start 117.61 50.9025) (end 117.61 51.255) (width 0.7) (layer "F.Cu") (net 23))
 (segment (start 124.37 52.415) (end 118.77 52.415) (width 0.7) (layer "F.Cu") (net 23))
 (segment (start 126.82 49.965) (end 124.37 52.415) (width 0.7) (layer "F.Cu") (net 23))
 (segment (start 118.77 52.415) (end 117.63 53.555) (width 0.7) (layer "F.Cu") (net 23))
 (segment (start 117.99 71.375) (end 120.85 71.375) (width 0.7) (layer "B.Cu") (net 24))
 (segment (start 124.51 67.715) (end 124.51 54.815) (width 0.7) (layer "B.Cu") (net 24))
 (segment (start 116.21 68.205) (end 116.21 69.595) (width 0.7) (layer "B.Cu") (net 24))
 (segment (start 120.85 71.375) (end 124.51 67.715) (width 0.7) (layer "B.Cu") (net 24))
 (segment (start 124.51 54.815) (end 126.82 52.505) (width 0.7) (layer "B.Cu") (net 24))
 (segment (start 116.21 69.595) (end 117.99 71.375) (width 0.7) (layer "B.Cu") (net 24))
 (segment (start 143.9875 63.895) (end 144.76 63.895) (width 0.7) (layer "F.Cu") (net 13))
 (segment (start 138.35 51.015) (end 138.35 62.375) (width 0.7) (layer "F.Cu") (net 13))
 (segment (start 123.87 71.045) (end 121.32 73.595) (width 0.7) (layer "F.Cu") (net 13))
 (segment (start 143.15 63.0575) (end 143.9875 63.895) (width 0.7) (layer "F.Cu") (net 13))
 (segment (start 121.32 73.595) (end 121.31 73.595) (width 0.7) (layer "F.Cu") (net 13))
 (segment (start 150.21 58.445) (end 150.21 55.225) (width 0.7) (layer "F.Cu") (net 13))
 (segment (start 117.66 64.1875) (end 120.7125 64.1875) (width 0.7) (layer "F.Cu") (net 13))
 (segment (start 172.3275 48) (end 171.33 48.9975) (width 0.7) (layer "F.Cu") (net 13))
 (segment (start 138.35 62.375) (end 139.89 63.915) (width 0.7) (layer "F.Cu") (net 13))
 (segment (start 171.33 48.9975) (end 169.9375 47.605) (width 0.7) (layer "F.Cu") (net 13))
 (segment (start 120.7125 64.1875) (end 123.87 67.345) (width 0.7) (layer "F.Cu") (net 13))
 (segment (start 134.76 47.425) (end 138.35 51.015) (width 0.7) (layer "F.Cu") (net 13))
 (segment (start 123.87 67.345) (end 123.87 71.045) (width 0.7) (layer "F.Cu") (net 13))
 (segment (start 142.2925 63.915) (end 143.15 63.0575) (width 0.7) (layer "F.Cu") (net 13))
 (segment (start 144.76 63.895) (end 150.21 58.445) (width 0.7) (layer "F.Cu") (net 13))
 (segment (start 175.12 48) (end 172.3275 48) (width 0.7) (layer "F.Cu") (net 13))
 (segment (start 139.89 63.915) (end 142.2925 63.915) (width 0.7) (layer "F.Cu") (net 13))
 (segment (start 169.9375 47.605) (end 158.15 47.605) (width 0.7) (layer "F.Cu") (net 13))
 (segment (start 178.53 61.415) (end 176.705 63.24) (width 0.7) (layer "B.Cu") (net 13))
 (segment (start 142.19 90.01) (end 142.19 80.86) (width 0.7) (layer "B.Cu") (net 13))
 (segment (start 126.82 68.085) (end 126.82 55.045) (width 0.7) (layer "B.Cu") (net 13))
 (segment (start 134.925 73.595) (end 121.31 73.595) (width 0.7) (layer "B.Cu") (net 13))
 (segment (start 178.53 49.825) (end 178.53 61.415) (width 0.7) (layer "B.Cu") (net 13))
 (segment (start 126.82 55.045) (end 134.44 47.425) (width 0.7) (layer "B.Cu") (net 13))
 (segment (start 121.31 73.595) (end 126.82 68.085) (width 0.7) (layer "B.Cu") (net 13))
 (segment (start 157.83 47.605) (end 158.15 47.605) (width 0.7) (layer "B.Cu") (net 13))
 (segment (start 175.12 48) (end 176.705 48) (width 0.7) (layer "B.Cu") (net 13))
 (segment (start 176.705 48) (end 178.53 49.825) (width 0.7) (layer "B.Cu") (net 13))
 (segment (start 134.44 47.425) (end 134.76 47.425) (width 0.7) (layer "B.Cu") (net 13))
 (segment (start 150.21 55.225) (end 157.83 47.605) (width 0.7) (layer "B.Cu") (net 13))
 (segment (start 152.75 105.905) (end 152.75 100.57) (width 0.7) (layer "B.Cu") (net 13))
 (segment (start 142.19 80.86) (end 134.925 73.595) (width 0.7) (layer "B.Cu") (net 13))
 (segment (start 152.75 100.57) (end 142.19 90.01) (width 0.7) (layer "B.Cu") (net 13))
 (segment (start 176.705 63.24) (end 175.12 63.24) (width 0.7) (layer "B.Cu") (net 13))
 (segment (start 152.72 50.145) (end 155.26 52.685) (width 0.7) (layer "F.Cu") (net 11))
 (segment (start 146.11 52.865) (end 144.3 52.865) (width 0.7) (layer "F.Cu") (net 11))
 (segment (start 144.3 52.865) (end 143.13 54.035) (width 0.7) (layer "F.Cu") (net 11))
 (segment (start 148.83 50.145) (end 146.11 52.865) (width 0.7) (layer "F.Cu") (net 11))
 (segment (start 150.21 50.145) (end 152.72 50.145) (width 0.7) (layer "F.Cu") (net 11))
 (segment (start 150.21 50.145) (end 148.83 50.145) (width 0.7) (layer "F.Cu") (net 11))
 (segment (start 155.26 52.685) (end 158.15 52.685) (width 0.7) (layer "F.Cu") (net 11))
 (segment (start 143.13 54.035) (end 143.13 54.3825) (width 0.7) (layer "F.Cu") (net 11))
 (segment (start 144.3 52.865) (end 143.11 51.675) (width 0.7) (layer "F.Cu") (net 11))
 (segment (start 147.25 80.105) (end 152.75 85.605) (width 0.7) (layer "B.Cu") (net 12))
 (segment (start 147.25 55.645) (end 147.25 80.105) (width 0.7) (layer "B.Cu") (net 12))
 (segment (start 150.21 52.685) (end 147.25 55.645) (width 0.7) (layer "B.Cu") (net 12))
 (segment (start 117.63 61.0325) (end 117.66 61.0625) (width 0.7) (layer "F.Cu") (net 18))
 (segment (start 117.63 57.3075) (end 117.63 61.0325) (width 0.7) (layer "F.Cu") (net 18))
 (segment (start 143.13 57.5075) (end 143.13 59.9125) (width 0.7) (layer "F.Cu") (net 16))
 (segment (start 143.13 59.9125) (end 143.15 59.9325) (width 0.7) (layer "F.Cu") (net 16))
 (segment (start 122.1 84.9675) (end 122.1 88.8325) (width 0.7) (layer "F.Cu") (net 4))
 (segment (start 117.57 87.9125) (end 121.18 87.9125) (width 0.7) (layer "F.Cu") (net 4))
 (segment (start 123.32 87.6125) (end 122.1 88.8325) (width 0.7) (layer "F.Cu") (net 4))
 (segment (start 116.59 88.8925) (end 117.57 87.9125) (width 0.7) (layer "F.Cu") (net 4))
 (segment (start 129.14 87.6125) (end 123.32 87.6125) (width 0.7) (layer "F.Cu") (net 4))
 (segment (start 121.18 87.9125) (end 122.1 88.8325) (width 0.7) (layer "F.Cu") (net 4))
 (segment (start 176.555 59.43) (end 178.52 61.395) (width 0.7) (layer "F.Cu") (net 8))
 (segment (start 178.52 69.725) (end 176.93 71.315) (width 0.7) (layer "F.Cu") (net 8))
 (segment (start 125.18 81.0525) (end 129.14 85.0125) (width 0.7) (layer "F.Cu") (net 8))
 (segment (start 139.87 85.025) (end 135.7175 85.025) (width 0.7) (layer "F.Cu") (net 8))
 (segment (start 122.1 81.8425) (end 122.89 81.0525) (width 0.7) (layer "F.Cu") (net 8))
 (segment (start 178.52 61.395) (end 178.52 69.725) (width 0.7) (layer "F.Cu") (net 8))
 (segment (start 153.58 71.315) (end 139.87 85.025) (width 0.7) (layer "F.Cu") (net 8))
 (segment (start 176.93 71.315) (end 153.58 71.315) (width 0.7) (layer "F.Cu") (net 8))
 (segment (start 135.7175 85.025) (end 134.55 86.1925) (width 0.7) (layer "F.Cu") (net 8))
 (segment (start 175.12 59.43) (end 176.555 59.43) (width 0.7) (layer "F.Cu") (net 8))
 (segment (start 122.89 81.0525) (end 125.18 81.0525) (width 0.7) (layer "F.Cu") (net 8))
 (segment (start 133.37 85.0125) (end 129.14 85.0125) (width 0.7) (layer "F.Cu") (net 8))
 (segment (start 134.55 86.1925) (end 133.37 85.0125) (width 0.7) (layer "F.Cu") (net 8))
 (segment (start 144.91 108.51) (end 148.71 112.31) (width 0.7) (layer "B.Cu") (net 5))
 (segment (start 148.71 112.31) (end 159.545 112.31) (width 0.7) (layer "B.Cu") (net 5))
 (segment (start 132.01 104.91) (end 132.01 103.2) (width 0.7) (layer "B.Cu") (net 5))
 (segment (start 132.01 120.955) (end 128.59 124.375) (width 0.7) (layer "B.Cu") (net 5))
 (segment (start 159.545 112.31) (end 170.165 101.69) (width 0.7) (layer "B.Cu") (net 5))
 (segment (start 144.91 105.19) (end 144.91 108.51) (width 0.7) (layer "B.Cu") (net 5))
 (segment (start 128.59 126.185) (end 128.59 124.375) (width 0.7) (layer "B.Cu") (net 5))
 (segment (start 132.01 104.91) (end 132.01 120.955) (width 0.7) (layer "B.Cu") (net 5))
 (segment (start 133.76 101.45) (end 141.17 101.45) (width 0.7) (layer "B.Cu") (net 5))
 (segment (start 141.17 101.45) (end 144.91 105.19) (width 0.7) (layer "B.Cu") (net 5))
 (segment (start 170.165 101.69) (end 173 101.69) (width 0.7) (layer "B.Cu") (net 5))
 (segment (start 132.01 103.2) (end 133.76 101.45) (width 0.7) (layer "B.Cu") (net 5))
 (segment (start 152.62 64.195) (end 153.74 65.315) (width 0.7) (layer "F.Cu") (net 1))
 (segment (start 164.85 69.645) (end 172.525 69.645) (width 0.7) (layer "F.Cu") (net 1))
 (segment (start 153.74 65.315) (end 157.66 65.315) (width 0.7) (layer "F.Cu") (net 1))
 (segment (start 164.29 69.085) (end 164.85 69.645) (width 0.7) (layer "F.Cu") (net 1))
 (segment (start 162.01 69.665) (end 157.66 65.315) (width 0.7) (layer "F.Cu") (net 1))
 (segment (start 172.525 69.645) (end 175.12 67.05) (width 0.7) (layer "F.Cu") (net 1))
 (segment (start 164.29 69.085) (end 163.71 69.665) (width 0.7) (layer "F.Cu") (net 1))
 (segment (start 163.71 69.665) (end 162.01 69.665) (width 0.7) (layer "F.Cu") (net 1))
 (segment (start 177.31 115.305) (end 171.73 109.725) (width 0.7) (layer "B.Cu") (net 9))
 (segment (start 171.73 109.725) (end 165.45 109.725) (width 0.7) (layer "B.Cu") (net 9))
 (segment (start 169.74 126.175) (end 177.31 118.605) (width 0.7) (layer "B.Cu") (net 9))
 (segment (start 158.46 126.175) (end 169.74 126.175) (width 0.7) (layer "B.Cu") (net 9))
 (segment (start 177.31 118.605) (end 177.31 115.305) (width 0.7) (layer "B.Cu") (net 9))
 (segment (start 173 94.07) (end 170.64 91.71) (width 0.7) (layer "F.Cu") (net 6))
 (segment (start 170.64 91.71) (end 170.64 87.175) (width 0.7) (layer "F.Cu") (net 6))
 (segment (start 170.64 87.175) (end 165.27 81.805) (width 0.7) (layer "F.Cu") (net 6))
 (segment (start 133.68 126.175) (end 133.67 126.185) (width 0.7) (layer "B.Cu") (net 7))
 (segment (start 153.38 126.175) (end 133.68 126.175) (width 0.7) (layer "B.Cu") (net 7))
 (segment (start 136.55 68.195) (end 150.75 68.195) (width 0.7) (layer "F.Cu") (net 17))
 (segment (start 116.21 73.605) (end 115.26 74.555) (width 0.7) (layer "F.Cu") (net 17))
 (segment (start 127.03 77.715) (end 136.55 68.195) (width 0.7) (layer "F.Cu") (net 17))
 (segment (start 115.26 76.785) (end 116.19 77.715) (width 0.7) (layer "F.Cu") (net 17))
 (segment (start 115.26 74.555) (end 115.26 76.785) (width 0.7) (layer "F.Cu") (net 17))
 (segment (start 116.19 77.715) (end 127.03 77.715) (width 0.7) (layer "F.Cu") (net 17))
 (via (at 150.75 68.195) (size 1) (drill 0.7) (layers "F.Cu" "B.Cu") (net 17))
 (segment (start 150.75 68.195) (end 162.545 68.195) (width 0.7) (layer "B.Cu") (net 17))
 (segment (start 162.545 68.195) (end 175.12 55.62) (width 0.7) (layer "B.Cu") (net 17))
 (segment (start 164.31 62.225) (end 164.31 65.94) (width 0.7) (layer "F.Cu") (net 2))
 (segment (start 164.31 65.94) (end 164.29 65.96) (width 0.7) (layer "F.Cu") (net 2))
 (segment (start 163.82 62.715) (end 157.66 62.715) (width 0.7) (layer "F.Cu") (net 2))
 (segment (start 164.31 62.225) (end 165.26 63.175) (width 0.7) (layer "F.Cu") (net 2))
 (segment (start 165.26 63.175) (end 169.07 63.175) (width 0.7) (layer "F.Cu") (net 2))
 (segment (start 169.07 63.175) (end 170.1 62.145) (width 0.7) (layer "F.Cu") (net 2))
 (segment (start 164.31 62.225) (end 163.82 62.715) (width 0.7) (layer "F.Cu") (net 2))
 (segment (start 137.09 109.88) (end 142.515 115.305) (width 0.7) (layer "B.Cu") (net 10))
 (segment (start 142.515 115.305) (end 172.23 115.305) (width 0.7) (layer "B.Cu") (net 10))
 (segment (start 137.09 104.91) (end 137.09 109.88) (width 0.7) (layer "B.Cu") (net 10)))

